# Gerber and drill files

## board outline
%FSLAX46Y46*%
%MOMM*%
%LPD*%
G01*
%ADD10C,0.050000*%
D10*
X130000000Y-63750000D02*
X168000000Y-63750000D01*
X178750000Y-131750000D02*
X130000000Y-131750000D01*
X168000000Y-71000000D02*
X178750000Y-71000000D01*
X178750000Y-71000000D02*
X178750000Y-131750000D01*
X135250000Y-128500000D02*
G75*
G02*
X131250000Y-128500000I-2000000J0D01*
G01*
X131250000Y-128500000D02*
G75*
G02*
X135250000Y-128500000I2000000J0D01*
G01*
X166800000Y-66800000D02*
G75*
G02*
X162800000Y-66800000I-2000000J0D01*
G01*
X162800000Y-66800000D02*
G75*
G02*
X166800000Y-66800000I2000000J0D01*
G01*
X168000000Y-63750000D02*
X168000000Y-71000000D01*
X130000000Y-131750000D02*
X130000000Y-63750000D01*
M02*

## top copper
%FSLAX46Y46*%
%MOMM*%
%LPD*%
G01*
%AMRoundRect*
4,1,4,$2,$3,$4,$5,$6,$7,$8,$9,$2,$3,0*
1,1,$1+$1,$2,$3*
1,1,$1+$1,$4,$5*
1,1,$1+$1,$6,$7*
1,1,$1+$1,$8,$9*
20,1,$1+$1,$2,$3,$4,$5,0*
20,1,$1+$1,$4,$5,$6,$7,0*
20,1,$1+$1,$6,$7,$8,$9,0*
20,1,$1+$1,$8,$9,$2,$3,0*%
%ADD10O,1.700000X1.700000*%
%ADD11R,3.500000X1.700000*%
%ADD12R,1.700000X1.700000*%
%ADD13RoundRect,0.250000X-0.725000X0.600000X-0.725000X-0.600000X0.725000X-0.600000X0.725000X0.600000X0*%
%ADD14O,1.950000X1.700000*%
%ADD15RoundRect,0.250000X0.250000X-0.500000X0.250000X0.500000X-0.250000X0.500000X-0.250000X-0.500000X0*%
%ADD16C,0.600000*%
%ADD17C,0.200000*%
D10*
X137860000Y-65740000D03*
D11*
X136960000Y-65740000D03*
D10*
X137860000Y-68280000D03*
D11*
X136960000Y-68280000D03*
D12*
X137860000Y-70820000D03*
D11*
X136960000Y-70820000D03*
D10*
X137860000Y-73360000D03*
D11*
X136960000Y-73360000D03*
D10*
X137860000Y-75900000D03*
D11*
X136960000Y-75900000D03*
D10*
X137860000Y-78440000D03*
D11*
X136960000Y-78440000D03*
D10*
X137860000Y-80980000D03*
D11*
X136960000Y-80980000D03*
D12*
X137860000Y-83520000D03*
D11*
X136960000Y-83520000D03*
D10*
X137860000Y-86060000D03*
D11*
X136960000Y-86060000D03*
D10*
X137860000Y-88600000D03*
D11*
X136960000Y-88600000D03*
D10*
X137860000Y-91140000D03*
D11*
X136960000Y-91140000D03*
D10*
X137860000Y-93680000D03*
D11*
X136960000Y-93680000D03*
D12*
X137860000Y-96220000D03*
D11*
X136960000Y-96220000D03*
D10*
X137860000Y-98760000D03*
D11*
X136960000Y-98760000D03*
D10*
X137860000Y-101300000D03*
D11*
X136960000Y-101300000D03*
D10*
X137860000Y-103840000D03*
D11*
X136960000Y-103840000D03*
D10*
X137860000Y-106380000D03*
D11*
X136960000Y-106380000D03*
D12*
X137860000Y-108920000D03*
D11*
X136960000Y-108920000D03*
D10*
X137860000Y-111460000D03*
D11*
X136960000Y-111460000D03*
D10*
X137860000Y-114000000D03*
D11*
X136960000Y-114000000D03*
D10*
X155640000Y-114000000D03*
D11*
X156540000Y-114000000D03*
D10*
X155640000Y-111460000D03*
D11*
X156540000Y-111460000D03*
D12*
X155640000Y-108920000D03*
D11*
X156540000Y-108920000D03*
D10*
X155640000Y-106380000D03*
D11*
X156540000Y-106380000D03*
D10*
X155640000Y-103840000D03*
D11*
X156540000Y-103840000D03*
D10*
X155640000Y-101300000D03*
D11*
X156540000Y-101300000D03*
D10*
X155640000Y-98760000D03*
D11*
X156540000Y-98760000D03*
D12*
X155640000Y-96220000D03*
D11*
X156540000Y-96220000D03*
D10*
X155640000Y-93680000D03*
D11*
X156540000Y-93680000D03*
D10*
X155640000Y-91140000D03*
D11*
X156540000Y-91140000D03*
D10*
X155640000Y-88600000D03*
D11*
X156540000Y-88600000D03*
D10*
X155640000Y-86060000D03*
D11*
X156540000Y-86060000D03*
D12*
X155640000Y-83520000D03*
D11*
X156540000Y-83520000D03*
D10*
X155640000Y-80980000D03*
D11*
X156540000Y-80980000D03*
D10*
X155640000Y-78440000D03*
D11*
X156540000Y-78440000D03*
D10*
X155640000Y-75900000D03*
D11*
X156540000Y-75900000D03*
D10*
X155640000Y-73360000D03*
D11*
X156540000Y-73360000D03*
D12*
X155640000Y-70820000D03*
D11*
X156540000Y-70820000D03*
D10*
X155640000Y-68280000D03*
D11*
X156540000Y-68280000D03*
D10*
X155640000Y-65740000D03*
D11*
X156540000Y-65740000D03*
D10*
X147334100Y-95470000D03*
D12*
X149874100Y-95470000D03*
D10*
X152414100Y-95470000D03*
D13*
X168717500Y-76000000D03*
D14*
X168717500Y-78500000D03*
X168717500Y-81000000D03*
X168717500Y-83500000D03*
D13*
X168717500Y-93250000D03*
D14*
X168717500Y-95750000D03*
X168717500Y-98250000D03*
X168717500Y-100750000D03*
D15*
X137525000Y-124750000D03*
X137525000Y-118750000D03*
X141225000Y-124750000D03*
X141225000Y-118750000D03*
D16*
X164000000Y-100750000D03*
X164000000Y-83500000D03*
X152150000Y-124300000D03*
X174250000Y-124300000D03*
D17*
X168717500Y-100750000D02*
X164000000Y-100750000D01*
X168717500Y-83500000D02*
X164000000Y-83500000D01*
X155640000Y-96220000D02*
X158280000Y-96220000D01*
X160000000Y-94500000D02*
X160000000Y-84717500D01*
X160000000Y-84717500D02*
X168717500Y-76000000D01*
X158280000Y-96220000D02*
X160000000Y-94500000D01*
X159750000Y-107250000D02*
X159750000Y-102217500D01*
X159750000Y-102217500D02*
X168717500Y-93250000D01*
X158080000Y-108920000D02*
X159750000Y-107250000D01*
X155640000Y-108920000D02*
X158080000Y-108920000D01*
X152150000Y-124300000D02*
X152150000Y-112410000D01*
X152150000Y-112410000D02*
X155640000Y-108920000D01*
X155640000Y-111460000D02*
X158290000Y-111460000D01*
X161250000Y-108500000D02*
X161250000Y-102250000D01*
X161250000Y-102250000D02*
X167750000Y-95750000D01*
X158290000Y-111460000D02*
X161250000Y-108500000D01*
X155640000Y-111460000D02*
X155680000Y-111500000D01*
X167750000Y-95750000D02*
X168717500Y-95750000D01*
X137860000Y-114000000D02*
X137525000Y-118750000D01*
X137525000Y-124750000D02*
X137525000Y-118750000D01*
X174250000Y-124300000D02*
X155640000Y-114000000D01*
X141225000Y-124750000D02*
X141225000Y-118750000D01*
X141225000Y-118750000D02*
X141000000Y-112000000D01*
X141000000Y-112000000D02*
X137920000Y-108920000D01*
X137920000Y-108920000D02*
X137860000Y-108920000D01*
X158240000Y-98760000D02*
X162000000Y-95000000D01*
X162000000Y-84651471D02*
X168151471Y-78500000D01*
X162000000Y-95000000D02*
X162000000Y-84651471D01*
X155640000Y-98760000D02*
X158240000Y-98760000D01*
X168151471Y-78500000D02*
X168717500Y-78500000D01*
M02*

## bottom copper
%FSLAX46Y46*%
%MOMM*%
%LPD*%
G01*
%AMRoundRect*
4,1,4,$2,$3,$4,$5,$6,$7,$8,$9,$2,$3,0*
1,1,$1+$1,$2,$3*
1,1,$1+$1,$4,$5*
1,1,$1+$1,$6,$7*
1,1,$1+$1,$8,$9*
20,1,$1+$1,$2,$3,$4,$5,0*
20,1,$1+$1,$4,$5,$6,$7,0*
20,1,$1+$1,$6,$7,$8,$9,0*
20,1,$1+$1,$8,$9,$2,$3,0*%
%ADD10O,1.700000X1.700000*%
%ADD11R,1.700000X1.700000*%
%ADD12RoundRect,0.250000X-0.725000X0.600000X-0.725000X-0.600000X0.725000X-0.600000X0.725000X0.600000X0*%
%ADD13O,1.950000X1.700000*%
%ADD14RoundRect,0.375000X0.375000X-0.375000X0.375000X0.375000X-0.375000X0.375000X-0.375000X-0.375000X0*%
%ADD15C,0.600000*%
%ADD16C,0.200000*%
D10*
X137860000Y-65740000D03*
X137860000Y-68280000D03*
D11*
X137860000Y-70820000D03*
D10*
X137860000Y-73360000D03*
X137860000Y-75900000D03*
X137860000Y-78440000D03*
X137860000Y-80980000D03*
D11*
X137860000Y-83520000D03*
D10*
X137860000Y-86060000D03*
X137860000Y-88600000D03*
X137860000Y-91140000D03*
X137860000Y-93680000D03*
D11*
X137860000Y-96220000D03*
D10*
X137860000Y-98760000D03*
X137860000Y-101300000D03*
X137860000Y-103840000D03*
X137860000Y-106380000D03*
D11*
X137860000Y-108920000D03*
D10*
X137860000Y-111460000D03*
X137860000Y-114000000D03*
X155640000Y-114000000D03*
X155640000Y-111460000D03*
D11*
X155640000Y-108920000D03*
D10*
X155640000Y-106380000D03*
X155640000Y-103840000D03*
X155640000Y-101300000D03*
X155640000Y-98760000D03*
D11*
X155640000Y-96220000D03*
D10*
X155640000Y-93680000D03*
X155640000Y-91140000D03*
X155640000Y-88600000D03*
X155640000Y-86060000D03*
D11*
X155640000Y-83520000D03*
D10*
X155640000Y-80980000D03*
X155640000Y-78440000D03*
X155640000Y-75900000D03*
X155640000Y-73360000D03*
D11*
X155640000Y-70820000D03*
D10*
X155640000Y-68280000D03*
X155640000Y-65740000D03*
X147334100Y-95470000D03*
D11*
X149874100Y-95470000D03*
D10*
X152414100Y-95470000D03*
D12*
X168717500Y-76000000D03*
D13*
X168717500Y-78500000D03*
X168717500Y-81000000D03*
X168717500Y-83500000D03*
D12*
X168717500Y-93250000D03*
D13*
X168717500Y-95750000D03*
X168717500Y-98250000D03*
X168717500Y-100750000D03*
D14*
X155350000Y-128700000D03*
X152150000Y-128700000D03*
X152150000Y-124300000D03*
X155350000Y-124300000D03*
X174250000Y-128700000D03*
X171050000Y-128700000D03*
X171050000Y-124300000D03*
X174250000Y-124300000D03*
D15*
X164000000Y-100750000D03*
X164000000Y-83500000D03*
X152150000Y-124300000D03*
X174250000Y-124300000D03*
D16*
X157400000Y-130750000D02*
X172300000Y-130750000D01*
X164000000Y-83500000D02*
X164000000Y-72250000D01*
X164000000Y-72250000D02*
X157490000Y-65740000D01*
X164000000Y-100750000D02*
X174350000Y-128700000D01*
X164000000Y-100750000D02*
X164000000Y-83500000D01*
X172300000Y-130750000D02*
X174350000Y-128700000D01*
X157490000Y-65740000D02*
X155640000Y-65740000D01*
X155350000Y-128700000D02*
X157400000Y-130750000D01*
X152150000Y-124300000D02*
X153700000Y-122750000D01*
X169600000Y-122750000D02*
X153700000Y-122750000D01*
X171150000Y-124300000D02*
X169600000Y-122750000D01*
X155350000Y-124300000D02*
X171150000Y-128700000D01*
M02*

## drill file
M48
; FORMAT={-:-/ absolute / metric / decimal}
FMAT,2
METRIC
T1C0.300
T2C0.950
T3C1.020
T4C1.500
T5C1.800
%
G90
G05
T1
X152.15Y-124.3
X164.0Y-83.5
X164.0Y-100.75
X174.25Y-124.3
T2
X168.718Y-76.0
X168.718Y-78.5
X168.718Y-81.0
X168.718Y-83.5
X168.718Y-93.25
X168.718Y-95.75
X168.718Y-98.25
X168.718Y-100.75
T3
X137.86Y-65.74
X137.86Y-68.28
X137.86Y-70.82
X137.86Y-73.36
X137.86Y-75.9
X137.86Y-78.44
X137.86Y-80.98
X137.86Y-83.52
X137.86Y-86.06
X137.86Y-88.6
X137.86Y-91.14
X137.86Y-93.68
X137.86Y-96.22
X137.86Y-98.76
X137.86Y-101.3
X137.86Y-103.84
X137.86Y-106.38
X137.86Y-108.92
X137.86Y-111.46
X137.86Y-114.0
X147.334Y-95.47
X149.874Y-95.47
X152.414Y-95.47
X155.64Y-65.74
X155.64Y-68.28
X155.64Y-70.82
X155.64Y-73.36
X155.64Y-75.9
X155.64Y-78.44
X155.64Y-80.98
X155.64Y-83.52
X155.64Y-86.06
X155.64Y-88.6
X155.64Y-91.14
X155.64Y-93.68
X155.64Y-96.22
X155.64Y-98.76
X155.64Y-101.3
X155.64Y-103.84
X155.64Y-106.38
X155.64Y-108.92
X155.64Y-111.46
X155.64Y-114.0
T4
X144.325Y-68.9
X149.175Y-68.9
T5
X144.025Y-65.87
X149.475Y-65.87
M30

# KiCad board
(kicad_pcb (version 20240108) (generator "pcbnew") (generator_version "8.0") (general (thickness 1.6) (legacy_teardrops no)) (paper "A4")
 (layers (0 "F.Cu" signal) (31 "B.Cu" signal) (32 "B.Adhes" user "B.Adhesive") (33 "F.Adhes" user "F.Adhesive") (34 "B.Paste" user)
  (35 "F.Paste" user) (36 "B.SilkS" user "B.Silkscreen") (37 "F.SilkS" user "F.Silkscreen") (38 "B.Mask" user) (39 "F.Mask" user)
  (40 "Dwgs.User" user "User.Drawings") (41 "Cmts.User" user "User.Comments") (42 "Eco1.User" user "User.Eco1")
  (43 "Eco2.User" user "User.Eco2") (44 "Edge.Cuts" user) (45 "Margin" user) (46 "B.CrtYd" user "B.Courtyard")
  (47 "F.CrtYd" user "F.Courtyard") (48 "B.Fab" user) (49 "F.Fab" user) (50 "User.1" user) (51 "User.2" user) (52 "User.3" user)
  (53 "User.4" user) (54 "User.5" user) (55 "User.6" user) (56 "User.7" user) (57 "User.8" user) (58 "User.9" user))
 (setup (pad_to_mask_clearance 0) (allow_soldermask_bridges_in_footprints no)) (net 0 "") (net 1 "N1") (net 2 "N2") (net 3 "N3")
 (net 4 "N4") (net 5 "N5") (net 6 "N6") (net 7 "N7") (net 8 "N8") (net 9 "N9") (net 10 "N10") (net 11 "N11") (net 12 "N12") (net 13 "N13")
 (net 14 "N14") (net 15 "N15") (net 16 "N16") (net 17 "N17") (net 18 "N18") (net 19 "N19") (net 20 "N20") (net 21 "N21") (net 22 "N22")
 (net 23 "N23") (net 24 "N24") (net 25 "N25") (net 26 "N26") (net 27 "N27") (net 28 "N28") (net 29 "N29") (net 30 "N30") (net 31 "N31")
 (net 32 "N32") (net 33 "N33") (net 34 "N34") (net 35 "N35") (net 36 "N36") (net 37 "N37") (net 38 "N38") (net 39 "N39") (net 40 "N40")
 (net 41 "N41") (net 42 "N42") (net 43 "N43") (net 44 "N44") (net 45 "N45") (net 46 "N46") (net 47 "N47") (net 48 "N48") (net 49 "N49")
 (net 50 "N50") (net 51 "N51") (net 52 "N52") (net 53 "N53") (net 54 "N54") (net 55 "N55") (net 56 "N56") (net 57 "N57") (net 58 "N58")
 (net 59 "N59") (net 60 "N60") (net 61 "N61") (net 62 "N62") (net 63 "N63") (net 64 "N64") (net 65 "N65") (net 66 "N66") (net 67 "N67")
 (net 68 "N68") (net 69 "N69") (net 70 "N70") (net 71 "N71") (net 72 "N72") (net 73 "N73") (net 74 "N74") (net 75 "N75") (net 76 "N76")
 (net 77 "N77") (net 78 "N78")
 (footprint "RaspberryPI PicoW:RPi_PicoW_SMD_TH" (layer "F.Cu") (at 146.75 89.87)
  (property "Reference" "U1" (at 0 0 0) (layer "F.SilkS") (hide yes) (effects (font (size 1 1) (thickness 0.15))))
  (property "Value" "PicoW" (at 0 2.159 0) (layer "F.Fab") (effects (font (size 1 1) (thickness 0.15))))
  (pad "" np_thru_hole oval (at -2.725 -24) (size 1.8 1.8) (drill 1.8) (layers "*.Cu" "*.Mask"))
  (pad "" np_thru_hole oval (at -2.425 -20.97) (size 1.5 1.5) (drill 1.5) (layers "*.Cu" "*.Mask"))
  (pad "" np_thru_hole oval (at 2.425 -20.97) (size 1.5 1.5) (drill 1.5) (layers "*.Cu" "*.Mask"))
  (pad "" np_thru_hole oval (at 2.725 -24) (size 1.8 1.8) (drill 1.8) (layers "*.Cu" "*.Mask"))
  (pad "1" thru_hole oval (at -8.89 -24.13) (size 1.7 1.7) (drill 1.02) (layers "*.Cu" "*.Mask") (remove_unused_layers no) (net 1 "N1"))
  (pad "1" smd rect (at -8.89 -24.13) (size 3.5 1.7) (drill (offset -0.9 0)) (layers "F.Cu" "F.Mask") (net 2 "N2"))
  (pad "2" thru_hole oval (at -8.89 -21.59) (size 1.7 1.7) (drill 1.02) (layers "*.Cu" "*.Mask") (remove_unused_layers no) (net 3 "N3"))
  (pad "2" smd rect (at -8.89 -21.59) (size 3.5 1.7) (drill (offset -0.9 0)) (layers "F.Cu" "F.Mask") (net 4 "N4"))
  (pad "3" thru_hole rect (at -8.89 -19.05) (size 1.7 1.7) (drill 1.02) (layers "*.Cu" "*.Mask") (remove_unused_layers no) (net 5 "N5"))
  (pad "3" smd rect (at -8.89 -19.05) (size 3.5 1.7) (drill (offset -0.9 0)) (layers "F.Cu" "F.Mask") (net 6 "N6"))
  (pad "4" thru_hole oval (at -8.89 -16.51) (size 1.7 1.7) (drill 1.02) (layers "*.Cu" "*.Mask") (remove_unused_layers no) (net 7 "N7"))
  (pad "4" smd rect (at -8.89 -16.51) (size 3.5 1.7) (drill (offset -0.9 0)) (layers "F.Cu" "F.Mask") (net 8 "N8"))
  (pad "5" thru_hole oval (at -8.89 -13.97) (size 1.7 1.7) (drill 1.02) (layers "*.Cu" "*.Mask") (remove_unused_layers no) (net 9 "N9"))
  (pad "5" smd rect (at -8.89 -13.97) (size 3.5 1.7) (drill (offset -0.9 0)) (layers "F.Cu" "F.Mask") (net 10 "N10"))
  (pad "6" thru_hole oval (at -8.89 -11.43) (size 1.7 1.7) (drill 1.02) (layers "*.Cu" "*.Mask") (remove_unused_layers no) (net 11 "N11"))
  (pad "6" smd rect (at -8.89 -11.43) (size 3.5 1.7) (drill (offset -0.9 0)) (layers "F.Cu" "F.Mask") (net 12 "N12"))
  (pad "7" thru_hole oval (at -8.89 -8.89) (size 1.7 1.7) (drill 1.02) (layers "*.Cu" "*.Mask") (remove_unused_layers no) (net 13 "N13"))
  (pad "7" smd rect (at -8.89 -8.89) (size 3.5 1.7) (drill (offset -0.9 0)) (layers "F.Cu" "F.Mask") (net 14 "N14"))
  (pad "8" thru_hole rect (at -8.89 -6.35) (size 1.7 1.7) (drill 1.02) (layers "*.Cu" "*.Mask") (remove_unused_layers no) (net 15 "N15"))
  (pad "8" smd rect (at -8.89 -6.35) (size 3.5 1.7) (drill (offset -0.9 0)) (layers "F.Cu" "F.Mask") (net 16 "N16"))
  (pad "9" thru_hole oval (at -8.89 -3.81) (size 1.7 1.7) (drill 1.02) (layers "*.Cu" "*.Mask") (remove_unused_layers no) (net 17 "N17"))
  (pad "9" smd rect (at -8.89 -3.81) (size 3.5 1.7) (drill (offset -0.9 0)) (layers "F.Cu" "F.Mask") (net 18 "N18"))
  (pad "10" thru_hole oval (at -8.89 -1.27) (size 1.7 1.7) (drill 1.02) (layers "*.Cu" "*.Mask") (remove_unused_layers no) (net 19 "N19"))
  (pad "10" smd rect (at -8.89 -1.27) (size 3.5 1.7) (drill (offset -0.9 0)) (layers "F.Cu" "F.Mask") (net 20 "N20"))
  (pad "11" thru_hole oval (at -8.89 1.27) (size 1.7 1.7) (drill 1.02) (layers "*.Cu" "*.Mask") (remove_unused_layers no) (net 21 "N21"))
  (pad "11" smd rect (at -8.89 1.27) (size 3.5 1.7) (drill (offset -0.9 0)) (layers "F.Cu" "F.Mask") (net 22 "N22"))
  (pad "12" thru_hole oval (at -8.89 3.81) (size 1.7 1.7) (drill 1.02) (layers "*.Cu" "*.Mask") (remove_unused_layers no) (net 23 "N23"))
  (pad "12" smd rect (at -8.89 3.81) (size 3.5 1.7) (drill (offset -0.9 0)) (layers "F.Cu" "F.Mask") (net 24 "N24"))
  (pad "13" thru_hole rect (at -8.89 6.35) (size 1.7 1.7) (drill 1.02) (layers "*.Cu" "*.Mask") (remove_unused_layers no) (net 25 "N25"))
  (pad "13" smd rect (at -8.89 6.35) (size 3.5 1.7) (drill (offset -0.9 0)) (layers "F.Cu" "F.Mask") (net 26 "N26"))
  (pad "14" thru_hole oval (at -8.89 8.89) (size 1.7 1.7) (drill 1.02) (layers "*.Cu" "*.Mask") (remove_unused_layers no) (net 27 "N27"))
  (pad "14" smd rect (at -8.89 8.89) (size 3.5 1.7) (drill (offset -0.9 0)) (layers "F.Cu" "F.Mask") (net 27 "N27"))
  (pad "15" thru_hole oval (at -8.89 11.43) (size 1.7 1.7) (drill 1.02) (layers "*.Cu" "*.Mask") (remove_unused_layers no) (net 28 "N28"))
  (pad "15" smd rect (at -8.89 11.43) (size 3.5 1.7) (drill (offset -0.9 0)) (layers "F.Cu" "F.Mask") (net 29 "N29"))
  (pad "16" thru_hole oval (at -8.89 13.97) (size 1.7 1.7) (drill 1.02) (layers "*.Cu" "*.Mask") (remove_unused_layers no) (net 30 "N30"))
  (pad "16" smd rect (at -8.89 13.97) (size 3.5 1.7) (drill (offset -0.9 0)) (layers "F.Cu" "F.Mask") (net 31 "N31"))
  (pad "17" thru_hole oval (at -8.89 16.51) (size 1.7 1.7) (drill 1.02) (layers "*.Cu" "*.Mask") (remove_unused_layers no) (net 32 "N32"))
  (pad "17" smd rect (at -8.89 16.51) (size 3.5 1.7) (drill (offset -0.9 0)) (layers "F.Cu" "F.Mask") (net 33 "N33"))
  (pad "18" thru_hole rect (at -8.89 19.05) (size 1.7 1.7) (drill 1.02) (layers "*.Cu" "*.Mask") (remove_unused_layers no) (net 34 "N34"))
  (pad "18" smd rect (at -8.89 19.05) (size 3.5 1.7) (drill (offset -0.9 0)) (layers "F.Cu" "F.Mask") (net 34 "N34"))
  (pad "19" thru_hole oval (at -8.89 21.59) (size 1.7 1.7) (drill 1.02) (layers "*.Cu" "*.Mask") (remove_unused_layers no) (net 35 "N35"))
  (pad "19" smd rect (at -8.89 21.59) (size 3.5 1.7) (drill (offset -0.9 0)) (layers "F.Cu" "F.Mask") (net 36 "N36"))
  (pad "20" thru_hole oval (at -8.89 24.13) (size 1.7 1.7) (drill 1.02) (layers "*.Cu" "*.Mask") (remove_unused_layers no) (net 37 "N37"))
  (pad "20" smd rect (at -8.89 24.13) (size 3.5 1.7) (drill (offset -0.9 0)) (layers "F.Cu" "F.Mask") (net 37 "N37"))
  (pad "21" thru_hole oval (at 8.89 24.13) (size 1.7 1.7) (drill 1.02) (layers "*.Cu" "*.Mask") (remove_unused_layers no) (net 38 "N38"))
  (pad "21" smd rect (at 8.89 24.13) (size 3.5 1.7) (drill (offset 0.9 0)) (layers "F.Cu" "F.Mask") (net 38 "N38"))
  (pad "22" thru_hole oval (at 8.89 21.59) (size 1.7 1.7) (drill 1.02) (layers "*.Cu" "*.Mask") (remove_unused_layers no) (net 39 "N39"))
  (pad "22" smd rect (at 8.89 21.59) (size 3.5 1.7) (drill (offset 0.9 0)) (layers "F.Cu" "F.Mask") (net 39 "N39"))
  (pad "23" thru_hole rect (at 8.89 19.05) (size 1.7 1.7) (drill 1.02) (layers "*.Cu" "*.Mask") (remove_unused_layers no) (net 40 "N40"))
  (pad "23" smd rect (at 8.89 19.05) (size 3.5 1.7) (drill (offset 0.9 0)) (layers "F.Cu" "F.Mask") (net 40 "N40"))
  (pad "24" thru_hole oval (at 8.89 16.51) (size 1.7 1.7) (drill 1.02) (layers "*.Cu" "*.Mask") (remove_unused_layers no) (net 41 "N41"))
  (pad "24" smd rect (at 8.89 16.51) (size 3.5 1.7) (drill (offset 0.9 0)) (layers "F.Cu" "F.Mask") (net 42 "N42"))
  (pad "25" thru_hole oval (at 8.89 13.97) (size 1.7 1.7) (drill 1.02) (layers "*.Cu" "*.Mask") (remove_unused_layers no) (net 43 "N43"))
  (pad "25" smd rect (at 8.89 13.97) (size 3.5 1.7) (drill (offset 0.9 0)) (layers "F.Cu" "F.Mask") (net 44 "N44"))
  (pad "26" thru_hole oval (at 8.89 11.43) (size 1.7 1.7) (drill 1.02) (layers "*.Cu" "*.Mask") (remove_unused_layers no) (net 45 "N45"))
  (pad "26" smd rect (at 8.89 11.43) (size 3.5 1.7) (drill (offset 0.9 0)) (layers "F.Cu" "F.Mask") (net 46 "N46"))
  (pad "27" thru_hole oval (at 8.89 8.89) (size 1.7 1.7) (drill 1.02) (layers "*.Cu" "*.Mask") (remove_unused_layers no) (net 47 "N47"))
  (pad "27" smd rect (at 8.89 8.89) (size 3.5 1.7) (drill (offset 0.9 0)) (layers "F.Cu" "F.Mask") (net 47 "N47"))
  (pad "28" thru_hole rect (at 8.89 6.35) (size 1.7 1.7) (drill 1.02) (layers "*.Cu" "*.Mask") (remove_unused_layers no) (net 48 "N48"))
  (pad "28" smd rect (at 8.89 6.35) (size 3.5 1.7) (drill (offset 0.9 0)) (layers "F.Cu" "F.Mask") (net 48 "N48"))
  (pad "29" thru_hole oval (at 8.89 3.81) (size 1.7 1.7) (drill 1.02) (layers "*.Cu" "*.Mask") (remove_unused_layers no) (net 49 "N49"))
  (pad "29" smd rect (at 8.89 3.81) (size 3.5 1.7) (drill (offset 0.9 0)) (layers "F.Cu" "F.Mask") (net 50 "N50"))
  (pad "30" thru_hole oval (at 8.89 1.27) (size 1.7 1.7) (drill 1.02) (layers "*.Cu" "*.Mask") (remove_unused_layers no) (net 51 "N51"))
  (pad "30" smd rect (at 8.89 1.27) (size 3.5 1.7) (drill (offset 0.9 0)) (layers "F.Cu" "F.Mask") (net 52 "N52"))
  (pad "31" thru_hole oval (at 8.89 -1.27) (size 1.7 1.7) (drill 1.02) (layers "*.Cu" "*.Mask") (remove_unused_layers no) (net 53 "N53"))
  (pad "31" smd rect (at 8.89 -1.27) (size 3.5 1.7) (drill (offset 0.9 0)) (layers "F.Cu" "F.Mask") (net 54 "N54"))
  (pad "32" thru_hole oval (at 8.89 -3.81) (size 1.7 1.7) (drill 1.02) (layers "*.Cu" "*.Mask") (remove_unused_layers no) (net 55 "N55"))
  (pad "32" smd rect (at 8.89 -3.81) (size 3.5 1.7) (drill (offset 0.9 0)) (layers "F.Cu" "F.Mask") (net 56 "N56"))
  (pad "33" thru_hole rect (at 8.89 -6.35) (size 1.7 1.7) (drill 1.02) (layers "*.Cu" "*.Mask") (remove_unused_layers no) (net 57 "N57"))
  (pad "33" smd rect (at 8.89 -6.35) (size 3.5 1.7) (drill (offset 0.9 0)) (layers "F.Cu" "F.Mask") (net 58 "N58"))
  (pad "34" thru_hole oval (at 8.89 -8.89) (size 1.7 1.7) (drill 1.02) (layers "*.Cu" "*.Mask") (remove_unused_layers no) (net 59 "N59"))
  (pad "34" smd rect (at 8.89 -8.89) (size 3.5 1.7) (drill (offset 0.9 0)) (layers "F.Cu" "F.Mask") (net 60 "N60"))
  (pad "35" thru_hole oval (at 8.89 -11.43) (size 1.7 1.7) (drill 1.02) (layers "*.Cu" "*.Mask") (remove_unused_layers no) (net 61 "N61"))
  (pad "35" smd rect (at 8.89 -11.43) (size 3.5 1.7) (drill (offset 0.9 0)) (layers "F.Cu" "F.Mask") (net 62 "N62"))
  (pad "36" thru_hole oval (at 8.89 -13.97) (size 1.7 1.7) (drill 1.02) (layers "*.Cu" "*.Mask") (remove_unused_layers no) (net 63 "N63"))
  (pad "36" smd rect (at 8.89 -13.97) (size 3.5 1.7) (drill (offset 0.9 0)) (layers "F.Cu" "F.Mask") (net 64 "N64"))
  (pad "37" thru_hole oval (at 8.89 -16.51) (size 1.7 1.7) (drill 1.02) (layers "*.Cu" "*.Mask") (remove_unused_layers no) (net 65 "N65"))
  (pad "37" smd rect (at 8.89 -16.51) (size 3.5 1.7) (drill (offset 0.9 0)) (layers "F.Cu" "F.Mask") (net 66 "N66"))
  (pad "38" thru_hole rect (at 8.89 -19.05) (size 1.7 1.7) (drill 1.02) (layers "*.Cu" "*.Mask") (remove_unused_layers no) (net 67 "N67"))
  (pad "38" smd rect (at 8.89 -19.05) (size 3.5 1.7) (drill (offset 0.9 0)) (layers "F.Cu" "F.Mask") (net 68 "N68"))
  (pad "39" thru_hole oval (at 8.89 -21.59) (size 1.7 1.7) (drill 1.02) (layers "*.Cu" "*.Mask") (remove_unused_layers no) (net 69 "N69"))
  (pad "39" smd rect (at 8.89 -21.59) (size 3.5 1.7) (drill (offset 0.9 0)) (layers "F.Cu" "F.Mask") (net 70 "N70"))
  (pad "40" thru_hole oval (at 8.89 -24.13) (size 1.7 1.7) (drill 1.02) (layers "*.Cu" "*.Mask") (remove_unused_layers no) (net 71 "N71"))
  (pad "40" smd rect (at 8.89 -24.13) (size 3.5 1.7) (drill (offset 0.9 0)) (layers "F.Cu" "F.Mask") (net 71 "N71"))
  (pad "41" thru_hole oval (at 0.5841 5.6) (size 1.7 1.7) (drill 1.02) (layers "*.Cu" "*.Mask") (remove_unused_layers no) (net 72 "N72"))
  (pad "42" thru_hole rect (at 3.1241 5.6) (size 1.7 1.7) (drill 1.02) (layers "*.Cu" "*.Mask") (remove_unused_layers no) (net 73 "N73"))
  (pad "43" thru_hole oval (at 5.6641 5.6) (size 1.7 1.7) (drill 1.02) (layers "*.Cu" "*.Mask") (remove_unused_layers no) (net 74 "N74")))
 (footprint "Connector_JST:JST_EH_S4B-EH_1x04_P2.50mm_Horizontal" (layer "F.Cu") (at 168.7175 76 -90)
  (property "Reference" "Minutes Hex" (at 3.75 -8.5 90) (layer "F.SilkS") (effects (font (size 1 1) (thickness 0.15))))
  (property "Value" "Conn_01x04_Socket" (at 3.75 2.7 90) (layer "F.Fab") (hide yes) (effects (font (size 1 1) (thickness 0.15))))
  (pad "1" thru_hole roundrect (at 0 0 270) (size 1.7 1.95) (drill 0.95) (layers "*.Cu" "*.Mask") (remove_unused_layers no)
   (roundrect_rratio 0.147059) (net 48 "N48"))
  (pad "2" thru_hole oval (at 2.5 0 270) (size 1.7 1.95) (drill 0.95) (layers "*.Cu" "*.Mask") (remove_unused_layers no) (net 47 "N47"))
  (pad "3" thru_hole oval (at 5 0 270) (size 1.7 1.95) (drill 0.95) (layers "*.Cu" "*.Mask") (remove_unused_layers no) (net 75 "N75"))
  (pad "4" thru_hole oval (at 7.5 0 270) (size 1.7 1.95) (drill 0.95) (layers "*.Cu" "*.Mask") (remove_unused_layers no) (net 71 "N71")))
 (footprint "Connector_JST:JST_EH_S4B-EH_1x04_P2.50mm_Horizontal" (layer "F.Cu") (at 168.7175 93.25 -90)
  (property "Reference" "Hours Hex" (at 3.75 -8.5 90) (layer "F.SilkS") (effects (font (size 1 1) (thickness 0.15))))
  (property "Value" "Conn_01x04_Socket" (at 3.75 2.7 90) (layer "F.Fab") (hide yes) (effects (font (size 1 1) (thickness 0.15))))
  (pad "1" thru_hole roundrect (at 0 0 270) (size 1.7 1.95) (drill 0.95) (layers "*.Cu" "*.Mask") (remove_unused_layers no)
   (roundrect_rratio 0.147059) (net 40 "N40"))
  (pad "2" thru_hole oval (at 2.5 0 270) (size 1.7 1.95) (drill 0.95) (layers "*.Cu" "*.Mask") (remove_unused_layers no) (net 39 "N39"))
  (pad "3" thru_hole oval (at 5 0 270) (size 1.7 1.95) (drill 0.95) (layers "*.Cu" "*.Mask") (remove_unused_layers no) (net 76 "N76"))
  (pad "4" thru_hole oval (at 7.5 0 270) (size 1.7 1.95) (drill 0.95) (layers "*.Cu" "*.Mask") (remove_unused_layers no) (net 71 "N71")))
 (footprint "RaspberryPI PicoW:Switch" (layer "F.Cu") (at 144.225 121.75 90)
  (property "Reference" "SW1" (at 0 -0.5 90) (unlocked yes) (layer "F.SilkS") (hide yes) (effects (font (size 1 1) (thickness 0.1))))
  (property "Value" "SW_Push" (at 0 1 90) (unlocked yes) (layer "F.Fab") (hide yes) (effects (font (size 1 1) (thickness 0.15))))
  (pad "1" smd roundrect (at -3 -6.7 90) (size 1.5 1) (layers "F.Cu" "F.Paste" "F.Mask") (roundrect_rratio 0.25) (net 37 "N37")
   (thermal_bridge_angle 45))
  (pad "1" smd roundrect (at 3 -6.7 90) (size 1.5 1) (layers "F.Cu" "F.Paste" "F.Mask") (roundrect_rratio 0.25) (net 37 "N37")
   (thermal_bridge_angle 45))
  (pad "2" smd roundrect (at -3 -3 90) (size 1.5 1) (layers "F.Cu" "F.Paste" "F.Mask") (roundrect_rratio 0.25) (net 34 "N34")
   (thermal_bridge_angle 45))
  (pad "2" smd roundrect (at 3 -3 90) (size 1.5 1) (layers "F.Cu" "F.Paste" "F.Mask") (roundrect_rratio 0.25) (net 34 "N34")
   (thermal_bridge_angle 45)))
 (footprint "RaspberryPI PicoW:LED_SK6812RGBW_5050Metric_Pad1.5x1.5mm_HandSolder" (layer "B.Cu") (at 153.75 126.5 90)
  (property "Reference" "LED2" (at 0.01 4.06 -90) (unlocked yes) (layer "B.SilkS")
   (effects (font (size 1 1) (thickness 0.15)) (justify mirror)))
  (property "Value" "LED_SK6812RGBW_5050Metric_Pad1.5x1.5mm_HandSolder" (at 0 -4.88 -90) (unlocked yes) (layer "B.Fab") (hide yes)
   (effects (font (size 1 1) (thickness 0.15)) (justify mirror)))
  (pad "1" smd roundrect (at -2.2 1.6 90) (size 1.5 1.5) (layers "B.Cu" "B.Paste" "B.Mask") (roundrect_rratio 0.25) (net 71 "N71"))
  (pad "2" smd roundrect (at -2.2 -1.6 90) (size 1.5 1.5) (layers "B.Cu" "B.Paste" "B.Mask") (roundrect_rratio 0.25) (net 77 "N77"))
  (pad "3" smd roundrect (at 2.2 -1.6 90) (size 1.5 1.5) (layers "B.Cu" "B.Paste" "B.Mask") (roundrect_rratio 0.25) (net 40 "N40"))
  (pad "4" smd roundrect (at 2.2 1.6 90) (size 1.5 1.5) (layers "B.Cu" "B.Paste" "B.Mask") (roundrect_rratio 0.25) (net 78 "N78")))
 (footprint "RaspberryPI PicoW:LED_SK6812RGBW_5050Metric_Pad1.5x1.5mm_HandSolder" (layer "B.Cu") (at 172.65 126.5 90)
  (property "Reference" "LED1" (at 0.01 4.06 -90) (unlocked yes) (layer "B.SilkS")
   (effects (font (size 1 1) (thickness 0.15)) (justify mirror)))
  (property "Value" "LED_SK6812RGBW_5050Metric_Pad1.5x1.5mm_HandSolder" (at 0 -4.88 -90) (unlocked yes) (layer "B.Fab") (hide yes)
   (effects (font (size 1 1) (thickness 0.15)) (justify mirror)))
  (pad "1" smd roundrect (at -2.2 1.6 90) (size 1.5 1.5) (layers "B.Cu" "B.Paste" "B.Mask") (roundrect_rratio 0.25) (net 71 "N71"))
  (pad "2" smd roundrect (at -2.2 -1.6 90) (size 1.5 1.5) (layers "B.Cu" "B.Paste" "B.Mask") (roundrect_rratio 0.25) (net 78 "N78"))
  (pad "3" smd roundrect (at 2.2 -1.6 90) (size 1.5 1.5) (layers "B.Cu" "B.Paste" "B.Mask") (roundrect_rratio 0.25) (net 40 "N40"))
  (pad "4" smd roundrect (at 2.2 1.6 90) (size 1.5 1.5) (layers "B.Cu" "B.Paste" "B.Mask") (roundrect_rratio 0.25) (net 38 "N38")))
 (gr_line (start 130 63.75) (end 168 63.75) (stroke (width 0.05) (type default)) (layer "Edge.Cuts"))
 (gr_line (start 178.75 131.75) (end 130 131.75) (stroke (width 0.05) (type default)) (layer "Edge.Cuts"))
 (gr_line (start 168 71) (end 178.75 71) (stroke (width 0.05) (type default)) (layer "Edge.Cuts"))
 (gr_line (start 178.75 71) (end 178.75 131.75) (stroke (width 0.05) (type default)) (layer "Edge.Cuts"))
 (gr_circle (center 133.25 128.5) (end 135.25 128.5) (stroke (width 0.05) (type default)) (fill none) (layer "Edge.Cuts"))
 (gr_circle (center 164.8 66.8) (end 166.8 66.8) (stroke (width 0.05) (type default)) (fill none) (layer "Edge.Cuts"))
 (gr_line (start 168 63.75) (end 168 71) (stroke (width 0.05) (type default)) (layer "Edge.Cuts"))
 (gr_line (start 130 131.75) (end 130 63.75) (stroke (width 0.05) (type default)) (layer "Edge.Cuts"))
 (segment (start 168.7175 100.75) (end 164 100.75) (width 0.2) (layer "F.Cu") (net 71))
 (segment (start 168.7175 83.5) (end 164 83.5) (width 0.2) (layer "F.Cu") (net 71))
 (via (at 164 100.75) (size 0.6) (drill 0.3) (layers "F.Cu" "B.Cu") (free yes) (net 71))
 (via (at 164 83.5) (size 0.6) (drill 0.3) (layers "F.Cu" "B.Cu") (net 71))
 (segment (start 157.4 130.75) (end 172.3 130.75) (width 0.2) (layer "B.Cu") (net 71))
 (segment (start 164 83.5) (end 164 72.25) (width 0.2) (layer "B.Cu") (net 71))
 (segment (start 164 72.25) (end 157.49 65.74) (width 0.2) (layer "B.Cu") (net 71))
 (segment (start 164 100.75) (end 174.35 128.7) (width 0.2) (layer "B.Cu") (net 71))
 (segment (start 164 100.75) (end 164 83.5) (width 0.2) (layer "B.Cu") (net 71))
 (segment (start 172.3 130.75) (end 174.35 128.7) (width 0.2) (layer "B.Cu") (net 71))
 (segment (start 157.49 65.74) (end 155.64 65.74) (width 0.2) (layer "B.Cu") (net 71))
 (segment (start 155.35 128.7) (end 157.4 130.75) (width 0.2) (layer "B.Cu") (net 71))
 (segment (start 155.64 96.22) (end 158.28 96.22) (width 0.2) (layer "F.Cu") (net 48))
 (segment (start 160 94.5) (end 160 84.7175) (width 0.2) (layer "F.Cu") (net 48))
 (segment (start 160 84.7175) (end 168.7175 76) (width 0.2) (layer "F.Cu") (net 48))
 (segment (start 158.28 96.22) (end 160 94.5) (width 0.2) (layer "F.Cu") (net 48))
 (segment (start 159.75 107.25) (end 159.75 102.2175) (width 0.2) (layer "F.Cu") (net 40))
 (segment (start 159.75 102.2175) (end 168.7175 93.25) (width 0.2) (layer "F.Cu") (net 40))
 (segment (start 158.08 108.92) (end 159.75 107.25) (width 0.2) (layer "F.Cu") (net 40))
 (segment (start 155.64 108.92) (end 158.08 108.92) (width 0.2) (layer "F.Cu") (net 40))
 (segment (start 152.15 124.3) (end 152.15 112.41) (width 0.2) (layer "F.Cu") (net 40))
 (segment (start 152.15 112.41) (end 155.64 108.92) (width 0.2) (layer "F.Cu") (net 40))
 (via (at 152.15 124.3) (size 0.6) (drill 0.3) (layers "F.Cu" "B.Cu") (free yes) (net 40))
 (segment (start 152.15 124.3) (end 153.7 122.75) (width 0.2) (layer "B.Cu") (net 40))
 (segment (start 169.6 122.75) (end 153.7 122.75) (width 0.2) (layer "B.Cu") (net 40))
 (segment (start 171.15 124.3) (end 169.6 122.75) (width 0.2) (layer "B.Cu") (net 40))
 (segment (start 155.64 111.46) (end 158.29 111.46) (width 0.2) (layer "F.Cu") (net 39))
 (segment (start 161.25 108.5) (end 161.25 102.25) (width 0.2) (layer "F.Cu") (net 39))
 (segment (start 161.25 102.25) (end 167.75 95.75) (width 0.2) (layer "F.Cu") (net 39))
 (segment (start 158.29 111.46) (end 161.25 108.5) (width 0.2) (layer "F.Cu") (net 39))
 (segment (start 155.64 111.46) (end 155.68 111.5) (width 0.2) (layer "F.Cu") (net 39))
 (segment (start 167.75 95.75) (end 168.7175 95.75) (width 0.2) (layer "F.Cu") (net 39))
 (segment (start 137.86 114) (end 137.525 118.75) (width 0.2) (layer "F.Cu") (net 37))
 (segment (start 137.525 124.75) (end 137.525 118.75) (width 0.2) (layer "F.Cu") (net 37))
 (segment (start 155.35 124.3) (end 171.15 128.7) (width 0.2) (layer "B.Cu") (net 78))
 (segment (start 174.25 124.3) (end 155.64 114) (width 0.2) (layer "F.Cu") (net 38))
 (via (at 174.25 124.3) (size 0.6) (drill 0.3) (layers "F.Cu" "B.Cu") (free yes) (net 38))
 (segment (start 141.225 124.75) (end 141.225 118.75) (width 0.2) (layer "F.Cu") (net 34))
 (segment (start 141.225 118.75) (end 141 112) (width 0.2) (layer "F.Cu") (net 34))
 (segment (start 141 112) (end 137.92 108.92) (width 0.2) (layer "F.Cu") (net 34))
 (segment (start 137.92 108.92) (end 137.86 108.92) (width 0.2) (layer "F.Cu") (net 34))
 (segment (start 158.24 98.76) (end 162 95) (width 0.2) (layer "F.Cu") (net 47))
 (segment (start 162 84.651471) (end 168.151471 78.5) (width 0.2) (layer "F.Cu") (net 47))
 (segment (start 162 95) (end 162 84.651471) (width 0.2) (layer "F.Cu") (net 47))
 (segment (start 155.64 98.76) (end 158.24 98.76) (width 0.2) (layer "F.Cu") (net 47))
 (segment (start 168.151471 78.5) (end 168.7175 78.5) (width 0.2) (layer "F.Cu") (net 47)))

